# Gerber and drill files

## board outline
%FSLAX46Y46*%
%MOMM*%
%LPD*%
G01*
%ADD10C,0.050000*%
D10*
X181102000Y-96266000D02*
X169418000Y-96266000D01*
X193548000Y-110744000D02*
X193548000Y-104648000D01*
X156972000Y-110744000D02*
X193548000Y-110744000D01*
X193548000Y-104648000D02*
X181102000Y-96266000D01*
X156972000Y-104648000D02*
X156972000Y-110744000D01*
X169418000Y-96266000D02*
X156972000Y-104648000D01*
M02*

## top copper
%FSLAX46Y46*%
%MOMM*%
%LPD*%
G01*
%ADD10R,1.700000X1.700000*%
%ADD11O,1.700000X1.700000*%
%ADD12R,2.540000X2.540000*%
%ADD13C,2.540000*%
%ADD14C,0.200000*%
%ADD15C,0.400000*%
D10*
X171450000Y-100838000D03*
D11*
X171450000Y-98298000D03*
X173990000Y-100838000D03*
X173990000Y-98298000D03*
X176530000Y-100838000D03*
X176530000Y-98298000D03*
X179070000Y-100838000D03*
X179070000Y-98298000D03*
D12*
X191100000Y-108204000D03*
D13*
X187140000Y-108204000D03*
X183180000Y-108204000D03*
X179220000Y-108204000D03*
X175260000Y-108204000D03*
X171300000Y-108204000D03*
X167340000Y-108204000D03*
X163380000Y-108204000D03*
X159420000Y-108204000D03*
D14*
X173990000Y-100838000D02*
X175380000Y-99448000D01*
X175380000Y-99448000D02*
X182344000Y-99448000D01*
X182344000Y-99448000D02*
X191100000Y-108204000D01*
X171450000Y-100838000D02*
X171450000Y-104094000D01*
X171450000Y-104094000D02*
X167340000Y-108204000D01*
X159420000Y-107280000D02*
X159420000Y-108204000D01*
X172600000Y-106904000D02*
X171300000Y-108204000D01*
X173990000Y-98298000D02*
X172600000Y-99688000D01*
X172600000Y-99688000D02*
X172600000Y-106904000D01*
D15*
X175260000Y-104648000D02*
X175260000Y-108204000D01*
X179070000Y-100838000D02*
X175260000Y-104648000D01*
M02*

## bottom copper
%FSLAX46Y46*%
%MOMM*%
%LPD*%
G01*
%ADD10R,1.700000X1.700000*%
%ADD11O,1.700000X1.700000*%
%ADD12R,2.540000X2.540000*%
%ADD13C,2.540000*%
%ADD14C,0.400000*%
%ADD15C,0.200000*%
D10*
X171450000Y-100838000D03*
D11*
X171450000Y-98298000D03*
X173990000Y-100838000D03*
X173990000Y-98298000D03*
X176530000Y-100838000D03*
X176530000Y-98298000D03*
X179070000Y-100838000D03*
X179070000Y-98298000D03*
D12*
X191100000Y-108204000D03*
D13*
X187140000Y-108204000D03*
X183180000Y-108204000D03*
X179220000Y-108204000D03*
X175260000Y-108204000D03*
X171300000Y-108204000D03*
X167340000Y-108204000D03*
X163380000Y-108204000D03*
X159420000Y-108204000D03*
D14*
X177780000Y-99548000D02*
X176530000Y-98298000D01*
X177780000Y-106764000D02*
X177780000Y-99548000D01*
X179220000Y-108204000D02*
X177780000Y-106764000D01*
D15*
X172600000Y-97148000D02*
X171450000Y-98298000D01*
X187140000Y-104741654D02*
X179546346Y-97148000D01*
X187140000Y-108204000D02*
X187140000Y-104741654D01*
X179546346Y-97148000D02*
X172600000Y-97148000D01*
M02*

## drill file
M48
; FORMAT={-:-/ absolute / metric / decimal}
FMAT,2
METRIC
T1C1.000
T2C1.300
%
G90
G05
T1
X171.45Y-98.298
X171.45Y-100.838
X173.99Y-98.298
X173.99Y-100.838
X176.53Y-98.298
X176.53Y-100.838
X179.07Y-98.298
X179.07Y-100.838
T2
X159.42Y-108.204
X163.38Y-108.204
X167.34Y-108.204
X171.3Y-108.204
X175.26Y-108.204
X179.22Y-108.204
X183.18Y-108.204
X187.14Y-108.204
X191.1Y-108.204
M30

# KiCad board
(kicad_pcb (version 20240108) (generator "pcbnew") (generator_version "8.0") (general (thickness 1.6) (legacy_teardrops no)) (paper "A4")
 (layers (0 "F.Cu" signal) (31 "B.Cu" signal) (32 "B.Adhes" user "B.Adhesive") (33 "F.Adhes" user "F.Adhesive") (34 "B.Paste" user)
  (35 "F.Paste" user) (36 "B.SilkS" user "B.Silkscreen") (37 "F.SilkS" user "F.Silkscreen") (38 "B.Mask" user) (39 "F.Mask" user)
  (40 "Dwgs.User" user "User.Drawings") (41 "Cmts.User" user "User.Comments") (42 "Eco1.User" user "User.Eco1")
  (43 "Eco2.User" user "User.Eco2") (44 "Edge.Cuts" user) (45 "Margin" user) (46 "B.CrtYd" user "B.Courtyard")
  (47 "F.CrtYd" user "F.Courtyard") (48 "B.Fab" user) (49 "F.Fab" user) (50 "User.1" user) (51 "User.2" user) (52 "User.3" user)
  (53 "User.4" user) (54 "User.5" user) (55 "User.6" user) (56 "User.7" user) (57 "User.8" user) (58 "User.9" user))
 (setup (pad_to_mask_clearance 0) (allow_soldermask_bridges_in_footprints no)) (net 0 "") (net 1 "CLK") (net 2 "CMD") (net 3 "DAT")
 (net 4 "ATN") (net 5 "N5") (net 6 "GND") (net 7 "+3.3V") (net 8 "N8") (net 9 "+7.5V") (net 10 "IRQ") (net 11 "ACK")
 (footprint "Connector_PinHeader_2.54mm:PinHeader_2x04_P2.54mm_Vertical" (layer "F.Cu") (at 171.45 100.838 90)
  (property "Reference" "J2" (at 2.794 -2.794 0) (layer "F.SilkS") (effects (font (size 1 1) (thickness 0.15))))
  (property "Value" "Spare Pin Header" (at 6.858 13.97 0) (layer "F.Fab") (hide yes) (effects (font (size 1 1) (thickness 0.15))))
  (pad "1" thru_hole rect (at 0 0 90) (size 1.7 1.7) (drill 1) (layers "*.Cu" "*.Mask") (remove_unused_layers no) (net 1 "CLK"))
  (pad "2" thru_hole oval (at 2.54 0 90) (size 1.7 1.7) (drill 1) (layers "*.Cu" "*.Mask") (remove_unused_layers no) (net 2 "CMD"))
  (pad "3" thru_hole oval (at 0 2.54 90) (size 1.7 1.7) (drill 1) (layers "*.Cu" "*.Mask") (remove_unused_layers no) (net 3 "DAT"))
  (pad "4" thru_hole oval (at 2.54 2.54 90) (size 1.7 1.7) (drill 1) (layers "*.Cu" "*.Mask") (remove_unused_layers no) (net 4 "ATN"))
  (pad "5" thru_hole oval (at 0 5.08 90) (size 1.7 1.7) (drill 1) (layers "*.Cu" "*.Mask") (remove_unused_layers no) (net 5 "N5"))
  (pad "6" thru_hole oval (at 2.54 5.08 90) (size 1.7 1.7) (drill 1) (layers "*.Cu" "*.Mask") (remove_unused_layers no) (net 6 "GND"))
  (pad "7" thru_hole oval (at 0 7.62 90) (size 1.7 1.7) (drill 1) (layers "*.Cu" "*.Mask") (remove_unused_layers no) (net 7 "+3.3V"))
  (pad "8" thru_hole oval (at 2.54 7.62 90) (size 1.7 1.7) (drill 1) (layers "*.Cu" "*.Mask") (remove_unused_layers no) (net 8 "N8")))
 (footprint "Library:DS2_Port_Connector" (layer "F.Cu") (at 175.26 108.204)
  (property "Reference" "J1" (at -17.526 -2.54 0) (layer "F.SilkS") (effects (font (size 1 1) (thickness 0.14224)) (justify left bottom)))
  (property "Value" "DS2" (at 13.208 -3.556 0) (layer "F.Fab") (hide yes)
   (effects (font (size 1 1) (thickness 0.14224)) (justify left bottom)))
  (pad "1" thru_hole rect (at 15.84 0) (size 2.54 2.54) (drill 1.3) (layers "*.Cu" "*.Mask") (remove_unused_layers no) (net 3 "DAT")
   (solder_mask_margin 0.0635))
  (pad "2" thru_hole circle (at 11.88 0) (size 2.54 2.54) (drill 1.3) (layers "*.Cu" "*.Mask") (remove_unused_layers no) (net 2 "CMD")
   (solder_mask_margin 0.0635))
  (pad "3" thru_hole circle (at 7.92 0) (size 2.54 2.54) (drill 1.3) (layers "*.Cu" "*.Mask") (remove_unused_layers no) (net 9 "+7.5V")
   (solder_mask_margin 0.0635))
  (pad "4" thru_hole circle (at 3.96 0) (size 2.54 2.54) (drill 1.3) (layers "*.Cu" "*.Mask") (remove_unused_layers no) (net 6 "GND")
   (solder_mask_margin 0.0635))
  (pad "5" thru_hole circle (at 0 0) (size 2.54 2.54) (drill 1.3) (layers "*.Cu" "*.Mask") (remove_unused_layers no) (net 7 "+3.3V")
   (solder_mask_margin 0.0635))
  (pad "6" thru_hole circle (at -3.96 0) (size 2.54 2.54) (drill 1.3) (layers "*.Cu" "*.Mask") (remove_unused_layers no) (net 4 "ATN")
   (solder_mask_margin 0.0635))
  (pad "7" thru_hole circle (at -7.92 0) (size 2.54 2.54) (drill 1.3) (layers "*.Cu" "*.Mask") (remove_unused_layers no) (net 1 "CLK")
   (solder_mask_margin 0.0635))
  (pad "8" thru_hole circle (at -11.88 0) (size 2.54 2.54) (drill 1.3) (layers "*.Cu" "*.Mask") (remove_unused_layers no) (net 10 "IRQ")
   (solder_mask_margin 0.0635))
  (pad "9" thru_hole circle (at -15.84 0 180) (size 2.54 2.54) (drill 1.3) (layers "*.Cu" "*.Mask") (remove_unused_layers no) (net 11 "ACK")
   (solder_mask_margin 0.0635)))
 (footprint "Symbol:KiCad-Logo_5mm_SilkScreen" (layer "B.Cu") (at 182.885698 104.657938 180)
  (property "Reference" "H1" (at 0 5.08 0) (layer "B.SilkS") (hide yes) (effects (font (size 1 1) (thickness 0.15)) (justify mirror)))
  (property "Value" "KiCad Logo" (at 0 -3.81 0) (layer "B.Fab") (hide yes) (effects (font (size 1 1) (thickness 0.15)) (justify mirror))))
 (gr_line (start 181.102 96.266) (end 169.418 96.266) (stroke (width 0.05) (type default)) (layer "Edge.Cuts"))
 (gr_line (start 193.548 110.744) (end 193.548 104.648) (stroke (width 0.05) (type default)) (layer "Edge.Cuts"))
 (gr_line (start 156.972 110.744) (end 193.548 110.744) (stroke (width 0.05) (type default)) (layer "Edge.Cuts"))
 (gr_line (start 193.548 104.648) (end 181.102 96.266) (stroke (width 0.05) (type default)) (layer "Edge.Cuts"))
 (gr_line (start 156.972 104.648) (end 156.972 110.744) (stroke (width 0.05) (type default)) (layer "Edge.Cuts"))
 (gr_line (start 169.418 96.266) (end 156.972 104.648) (stroke (width 0.05) (type default)) (layer "Edge.Cuts"))
 (segment (start 177.78 99.548) (end 176.53 98.298) (width 0.4) (layer "B.Cu") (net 6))
 (segment (start 177.78 106.764) (end 177.78 99.548) (width 0.4) (layer "B.Cu") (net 6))
 (segment (start 179.22 108.204) (end 177.78 106.764) (width 0.4) (layer "B.Cu") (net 6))
 (segment (start 173.99 100.838) (end 175.38 99.448) (width 0.2) (layer "F.Cu") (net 3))
 (segment (start 175.38 99.448) (end 182.344 99.448) (width 0.2) (layer "F.Cu") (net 3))
 (segment (start 182.344 99.448) (end 191.1 108.204) (width 0.2) (layer "F.Cu") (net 3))
 (segment (start 172.6 97.148) (end 171.45 98.298) (width 0.2) (layer "B.Cu") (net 2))
 (segment (start 187.14 104.741654) (end 179.546346 97.148) (width 0.2) (layer "B.Cu") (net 2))
 (segment (start 187.14 108.204) (end 187.14 104.741654) (width 0.2) (layer "B.Cu") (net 2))
 (segment (start 179.546346 97.148) (end 172.6 97.148) (width 0.2) (layer "B.Cu") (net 2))
 (segment (start 171.45 100.838) (end 171.45 104.094) (width 0.2) (layer "F.Cu") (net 1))
 (segment (start 171.45 104.094) (end 167.34 108.204) (width 0.2) (layer "F.Cu") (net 1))
 (segment (start 159.42 107.28) (end 159.42 108.204) (width 0.2) (layer "F.Cu") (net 11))
 (segment (start 172.6 106.904) (end 171.3 108.204) (width 0.2) (layer "F.Cu") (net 4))
 (segment (start 173.99 98.298) (end 172.6 99.688) (width 0.2) (layer "F.Cu") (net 4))
 (segment (start 172.6 99.688) (end 172.6 106.904) (width 0.2) (layer "F.Cu") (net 4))
 (segment (start 175.26 104.648) (end 175.26 108.204) (width 0.4) (layer "F.Cu") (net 7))
 (segment (start 179.07 100.838) (end 175.26 104.648) (width 0.4) (layer "F.Cu") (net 7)))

